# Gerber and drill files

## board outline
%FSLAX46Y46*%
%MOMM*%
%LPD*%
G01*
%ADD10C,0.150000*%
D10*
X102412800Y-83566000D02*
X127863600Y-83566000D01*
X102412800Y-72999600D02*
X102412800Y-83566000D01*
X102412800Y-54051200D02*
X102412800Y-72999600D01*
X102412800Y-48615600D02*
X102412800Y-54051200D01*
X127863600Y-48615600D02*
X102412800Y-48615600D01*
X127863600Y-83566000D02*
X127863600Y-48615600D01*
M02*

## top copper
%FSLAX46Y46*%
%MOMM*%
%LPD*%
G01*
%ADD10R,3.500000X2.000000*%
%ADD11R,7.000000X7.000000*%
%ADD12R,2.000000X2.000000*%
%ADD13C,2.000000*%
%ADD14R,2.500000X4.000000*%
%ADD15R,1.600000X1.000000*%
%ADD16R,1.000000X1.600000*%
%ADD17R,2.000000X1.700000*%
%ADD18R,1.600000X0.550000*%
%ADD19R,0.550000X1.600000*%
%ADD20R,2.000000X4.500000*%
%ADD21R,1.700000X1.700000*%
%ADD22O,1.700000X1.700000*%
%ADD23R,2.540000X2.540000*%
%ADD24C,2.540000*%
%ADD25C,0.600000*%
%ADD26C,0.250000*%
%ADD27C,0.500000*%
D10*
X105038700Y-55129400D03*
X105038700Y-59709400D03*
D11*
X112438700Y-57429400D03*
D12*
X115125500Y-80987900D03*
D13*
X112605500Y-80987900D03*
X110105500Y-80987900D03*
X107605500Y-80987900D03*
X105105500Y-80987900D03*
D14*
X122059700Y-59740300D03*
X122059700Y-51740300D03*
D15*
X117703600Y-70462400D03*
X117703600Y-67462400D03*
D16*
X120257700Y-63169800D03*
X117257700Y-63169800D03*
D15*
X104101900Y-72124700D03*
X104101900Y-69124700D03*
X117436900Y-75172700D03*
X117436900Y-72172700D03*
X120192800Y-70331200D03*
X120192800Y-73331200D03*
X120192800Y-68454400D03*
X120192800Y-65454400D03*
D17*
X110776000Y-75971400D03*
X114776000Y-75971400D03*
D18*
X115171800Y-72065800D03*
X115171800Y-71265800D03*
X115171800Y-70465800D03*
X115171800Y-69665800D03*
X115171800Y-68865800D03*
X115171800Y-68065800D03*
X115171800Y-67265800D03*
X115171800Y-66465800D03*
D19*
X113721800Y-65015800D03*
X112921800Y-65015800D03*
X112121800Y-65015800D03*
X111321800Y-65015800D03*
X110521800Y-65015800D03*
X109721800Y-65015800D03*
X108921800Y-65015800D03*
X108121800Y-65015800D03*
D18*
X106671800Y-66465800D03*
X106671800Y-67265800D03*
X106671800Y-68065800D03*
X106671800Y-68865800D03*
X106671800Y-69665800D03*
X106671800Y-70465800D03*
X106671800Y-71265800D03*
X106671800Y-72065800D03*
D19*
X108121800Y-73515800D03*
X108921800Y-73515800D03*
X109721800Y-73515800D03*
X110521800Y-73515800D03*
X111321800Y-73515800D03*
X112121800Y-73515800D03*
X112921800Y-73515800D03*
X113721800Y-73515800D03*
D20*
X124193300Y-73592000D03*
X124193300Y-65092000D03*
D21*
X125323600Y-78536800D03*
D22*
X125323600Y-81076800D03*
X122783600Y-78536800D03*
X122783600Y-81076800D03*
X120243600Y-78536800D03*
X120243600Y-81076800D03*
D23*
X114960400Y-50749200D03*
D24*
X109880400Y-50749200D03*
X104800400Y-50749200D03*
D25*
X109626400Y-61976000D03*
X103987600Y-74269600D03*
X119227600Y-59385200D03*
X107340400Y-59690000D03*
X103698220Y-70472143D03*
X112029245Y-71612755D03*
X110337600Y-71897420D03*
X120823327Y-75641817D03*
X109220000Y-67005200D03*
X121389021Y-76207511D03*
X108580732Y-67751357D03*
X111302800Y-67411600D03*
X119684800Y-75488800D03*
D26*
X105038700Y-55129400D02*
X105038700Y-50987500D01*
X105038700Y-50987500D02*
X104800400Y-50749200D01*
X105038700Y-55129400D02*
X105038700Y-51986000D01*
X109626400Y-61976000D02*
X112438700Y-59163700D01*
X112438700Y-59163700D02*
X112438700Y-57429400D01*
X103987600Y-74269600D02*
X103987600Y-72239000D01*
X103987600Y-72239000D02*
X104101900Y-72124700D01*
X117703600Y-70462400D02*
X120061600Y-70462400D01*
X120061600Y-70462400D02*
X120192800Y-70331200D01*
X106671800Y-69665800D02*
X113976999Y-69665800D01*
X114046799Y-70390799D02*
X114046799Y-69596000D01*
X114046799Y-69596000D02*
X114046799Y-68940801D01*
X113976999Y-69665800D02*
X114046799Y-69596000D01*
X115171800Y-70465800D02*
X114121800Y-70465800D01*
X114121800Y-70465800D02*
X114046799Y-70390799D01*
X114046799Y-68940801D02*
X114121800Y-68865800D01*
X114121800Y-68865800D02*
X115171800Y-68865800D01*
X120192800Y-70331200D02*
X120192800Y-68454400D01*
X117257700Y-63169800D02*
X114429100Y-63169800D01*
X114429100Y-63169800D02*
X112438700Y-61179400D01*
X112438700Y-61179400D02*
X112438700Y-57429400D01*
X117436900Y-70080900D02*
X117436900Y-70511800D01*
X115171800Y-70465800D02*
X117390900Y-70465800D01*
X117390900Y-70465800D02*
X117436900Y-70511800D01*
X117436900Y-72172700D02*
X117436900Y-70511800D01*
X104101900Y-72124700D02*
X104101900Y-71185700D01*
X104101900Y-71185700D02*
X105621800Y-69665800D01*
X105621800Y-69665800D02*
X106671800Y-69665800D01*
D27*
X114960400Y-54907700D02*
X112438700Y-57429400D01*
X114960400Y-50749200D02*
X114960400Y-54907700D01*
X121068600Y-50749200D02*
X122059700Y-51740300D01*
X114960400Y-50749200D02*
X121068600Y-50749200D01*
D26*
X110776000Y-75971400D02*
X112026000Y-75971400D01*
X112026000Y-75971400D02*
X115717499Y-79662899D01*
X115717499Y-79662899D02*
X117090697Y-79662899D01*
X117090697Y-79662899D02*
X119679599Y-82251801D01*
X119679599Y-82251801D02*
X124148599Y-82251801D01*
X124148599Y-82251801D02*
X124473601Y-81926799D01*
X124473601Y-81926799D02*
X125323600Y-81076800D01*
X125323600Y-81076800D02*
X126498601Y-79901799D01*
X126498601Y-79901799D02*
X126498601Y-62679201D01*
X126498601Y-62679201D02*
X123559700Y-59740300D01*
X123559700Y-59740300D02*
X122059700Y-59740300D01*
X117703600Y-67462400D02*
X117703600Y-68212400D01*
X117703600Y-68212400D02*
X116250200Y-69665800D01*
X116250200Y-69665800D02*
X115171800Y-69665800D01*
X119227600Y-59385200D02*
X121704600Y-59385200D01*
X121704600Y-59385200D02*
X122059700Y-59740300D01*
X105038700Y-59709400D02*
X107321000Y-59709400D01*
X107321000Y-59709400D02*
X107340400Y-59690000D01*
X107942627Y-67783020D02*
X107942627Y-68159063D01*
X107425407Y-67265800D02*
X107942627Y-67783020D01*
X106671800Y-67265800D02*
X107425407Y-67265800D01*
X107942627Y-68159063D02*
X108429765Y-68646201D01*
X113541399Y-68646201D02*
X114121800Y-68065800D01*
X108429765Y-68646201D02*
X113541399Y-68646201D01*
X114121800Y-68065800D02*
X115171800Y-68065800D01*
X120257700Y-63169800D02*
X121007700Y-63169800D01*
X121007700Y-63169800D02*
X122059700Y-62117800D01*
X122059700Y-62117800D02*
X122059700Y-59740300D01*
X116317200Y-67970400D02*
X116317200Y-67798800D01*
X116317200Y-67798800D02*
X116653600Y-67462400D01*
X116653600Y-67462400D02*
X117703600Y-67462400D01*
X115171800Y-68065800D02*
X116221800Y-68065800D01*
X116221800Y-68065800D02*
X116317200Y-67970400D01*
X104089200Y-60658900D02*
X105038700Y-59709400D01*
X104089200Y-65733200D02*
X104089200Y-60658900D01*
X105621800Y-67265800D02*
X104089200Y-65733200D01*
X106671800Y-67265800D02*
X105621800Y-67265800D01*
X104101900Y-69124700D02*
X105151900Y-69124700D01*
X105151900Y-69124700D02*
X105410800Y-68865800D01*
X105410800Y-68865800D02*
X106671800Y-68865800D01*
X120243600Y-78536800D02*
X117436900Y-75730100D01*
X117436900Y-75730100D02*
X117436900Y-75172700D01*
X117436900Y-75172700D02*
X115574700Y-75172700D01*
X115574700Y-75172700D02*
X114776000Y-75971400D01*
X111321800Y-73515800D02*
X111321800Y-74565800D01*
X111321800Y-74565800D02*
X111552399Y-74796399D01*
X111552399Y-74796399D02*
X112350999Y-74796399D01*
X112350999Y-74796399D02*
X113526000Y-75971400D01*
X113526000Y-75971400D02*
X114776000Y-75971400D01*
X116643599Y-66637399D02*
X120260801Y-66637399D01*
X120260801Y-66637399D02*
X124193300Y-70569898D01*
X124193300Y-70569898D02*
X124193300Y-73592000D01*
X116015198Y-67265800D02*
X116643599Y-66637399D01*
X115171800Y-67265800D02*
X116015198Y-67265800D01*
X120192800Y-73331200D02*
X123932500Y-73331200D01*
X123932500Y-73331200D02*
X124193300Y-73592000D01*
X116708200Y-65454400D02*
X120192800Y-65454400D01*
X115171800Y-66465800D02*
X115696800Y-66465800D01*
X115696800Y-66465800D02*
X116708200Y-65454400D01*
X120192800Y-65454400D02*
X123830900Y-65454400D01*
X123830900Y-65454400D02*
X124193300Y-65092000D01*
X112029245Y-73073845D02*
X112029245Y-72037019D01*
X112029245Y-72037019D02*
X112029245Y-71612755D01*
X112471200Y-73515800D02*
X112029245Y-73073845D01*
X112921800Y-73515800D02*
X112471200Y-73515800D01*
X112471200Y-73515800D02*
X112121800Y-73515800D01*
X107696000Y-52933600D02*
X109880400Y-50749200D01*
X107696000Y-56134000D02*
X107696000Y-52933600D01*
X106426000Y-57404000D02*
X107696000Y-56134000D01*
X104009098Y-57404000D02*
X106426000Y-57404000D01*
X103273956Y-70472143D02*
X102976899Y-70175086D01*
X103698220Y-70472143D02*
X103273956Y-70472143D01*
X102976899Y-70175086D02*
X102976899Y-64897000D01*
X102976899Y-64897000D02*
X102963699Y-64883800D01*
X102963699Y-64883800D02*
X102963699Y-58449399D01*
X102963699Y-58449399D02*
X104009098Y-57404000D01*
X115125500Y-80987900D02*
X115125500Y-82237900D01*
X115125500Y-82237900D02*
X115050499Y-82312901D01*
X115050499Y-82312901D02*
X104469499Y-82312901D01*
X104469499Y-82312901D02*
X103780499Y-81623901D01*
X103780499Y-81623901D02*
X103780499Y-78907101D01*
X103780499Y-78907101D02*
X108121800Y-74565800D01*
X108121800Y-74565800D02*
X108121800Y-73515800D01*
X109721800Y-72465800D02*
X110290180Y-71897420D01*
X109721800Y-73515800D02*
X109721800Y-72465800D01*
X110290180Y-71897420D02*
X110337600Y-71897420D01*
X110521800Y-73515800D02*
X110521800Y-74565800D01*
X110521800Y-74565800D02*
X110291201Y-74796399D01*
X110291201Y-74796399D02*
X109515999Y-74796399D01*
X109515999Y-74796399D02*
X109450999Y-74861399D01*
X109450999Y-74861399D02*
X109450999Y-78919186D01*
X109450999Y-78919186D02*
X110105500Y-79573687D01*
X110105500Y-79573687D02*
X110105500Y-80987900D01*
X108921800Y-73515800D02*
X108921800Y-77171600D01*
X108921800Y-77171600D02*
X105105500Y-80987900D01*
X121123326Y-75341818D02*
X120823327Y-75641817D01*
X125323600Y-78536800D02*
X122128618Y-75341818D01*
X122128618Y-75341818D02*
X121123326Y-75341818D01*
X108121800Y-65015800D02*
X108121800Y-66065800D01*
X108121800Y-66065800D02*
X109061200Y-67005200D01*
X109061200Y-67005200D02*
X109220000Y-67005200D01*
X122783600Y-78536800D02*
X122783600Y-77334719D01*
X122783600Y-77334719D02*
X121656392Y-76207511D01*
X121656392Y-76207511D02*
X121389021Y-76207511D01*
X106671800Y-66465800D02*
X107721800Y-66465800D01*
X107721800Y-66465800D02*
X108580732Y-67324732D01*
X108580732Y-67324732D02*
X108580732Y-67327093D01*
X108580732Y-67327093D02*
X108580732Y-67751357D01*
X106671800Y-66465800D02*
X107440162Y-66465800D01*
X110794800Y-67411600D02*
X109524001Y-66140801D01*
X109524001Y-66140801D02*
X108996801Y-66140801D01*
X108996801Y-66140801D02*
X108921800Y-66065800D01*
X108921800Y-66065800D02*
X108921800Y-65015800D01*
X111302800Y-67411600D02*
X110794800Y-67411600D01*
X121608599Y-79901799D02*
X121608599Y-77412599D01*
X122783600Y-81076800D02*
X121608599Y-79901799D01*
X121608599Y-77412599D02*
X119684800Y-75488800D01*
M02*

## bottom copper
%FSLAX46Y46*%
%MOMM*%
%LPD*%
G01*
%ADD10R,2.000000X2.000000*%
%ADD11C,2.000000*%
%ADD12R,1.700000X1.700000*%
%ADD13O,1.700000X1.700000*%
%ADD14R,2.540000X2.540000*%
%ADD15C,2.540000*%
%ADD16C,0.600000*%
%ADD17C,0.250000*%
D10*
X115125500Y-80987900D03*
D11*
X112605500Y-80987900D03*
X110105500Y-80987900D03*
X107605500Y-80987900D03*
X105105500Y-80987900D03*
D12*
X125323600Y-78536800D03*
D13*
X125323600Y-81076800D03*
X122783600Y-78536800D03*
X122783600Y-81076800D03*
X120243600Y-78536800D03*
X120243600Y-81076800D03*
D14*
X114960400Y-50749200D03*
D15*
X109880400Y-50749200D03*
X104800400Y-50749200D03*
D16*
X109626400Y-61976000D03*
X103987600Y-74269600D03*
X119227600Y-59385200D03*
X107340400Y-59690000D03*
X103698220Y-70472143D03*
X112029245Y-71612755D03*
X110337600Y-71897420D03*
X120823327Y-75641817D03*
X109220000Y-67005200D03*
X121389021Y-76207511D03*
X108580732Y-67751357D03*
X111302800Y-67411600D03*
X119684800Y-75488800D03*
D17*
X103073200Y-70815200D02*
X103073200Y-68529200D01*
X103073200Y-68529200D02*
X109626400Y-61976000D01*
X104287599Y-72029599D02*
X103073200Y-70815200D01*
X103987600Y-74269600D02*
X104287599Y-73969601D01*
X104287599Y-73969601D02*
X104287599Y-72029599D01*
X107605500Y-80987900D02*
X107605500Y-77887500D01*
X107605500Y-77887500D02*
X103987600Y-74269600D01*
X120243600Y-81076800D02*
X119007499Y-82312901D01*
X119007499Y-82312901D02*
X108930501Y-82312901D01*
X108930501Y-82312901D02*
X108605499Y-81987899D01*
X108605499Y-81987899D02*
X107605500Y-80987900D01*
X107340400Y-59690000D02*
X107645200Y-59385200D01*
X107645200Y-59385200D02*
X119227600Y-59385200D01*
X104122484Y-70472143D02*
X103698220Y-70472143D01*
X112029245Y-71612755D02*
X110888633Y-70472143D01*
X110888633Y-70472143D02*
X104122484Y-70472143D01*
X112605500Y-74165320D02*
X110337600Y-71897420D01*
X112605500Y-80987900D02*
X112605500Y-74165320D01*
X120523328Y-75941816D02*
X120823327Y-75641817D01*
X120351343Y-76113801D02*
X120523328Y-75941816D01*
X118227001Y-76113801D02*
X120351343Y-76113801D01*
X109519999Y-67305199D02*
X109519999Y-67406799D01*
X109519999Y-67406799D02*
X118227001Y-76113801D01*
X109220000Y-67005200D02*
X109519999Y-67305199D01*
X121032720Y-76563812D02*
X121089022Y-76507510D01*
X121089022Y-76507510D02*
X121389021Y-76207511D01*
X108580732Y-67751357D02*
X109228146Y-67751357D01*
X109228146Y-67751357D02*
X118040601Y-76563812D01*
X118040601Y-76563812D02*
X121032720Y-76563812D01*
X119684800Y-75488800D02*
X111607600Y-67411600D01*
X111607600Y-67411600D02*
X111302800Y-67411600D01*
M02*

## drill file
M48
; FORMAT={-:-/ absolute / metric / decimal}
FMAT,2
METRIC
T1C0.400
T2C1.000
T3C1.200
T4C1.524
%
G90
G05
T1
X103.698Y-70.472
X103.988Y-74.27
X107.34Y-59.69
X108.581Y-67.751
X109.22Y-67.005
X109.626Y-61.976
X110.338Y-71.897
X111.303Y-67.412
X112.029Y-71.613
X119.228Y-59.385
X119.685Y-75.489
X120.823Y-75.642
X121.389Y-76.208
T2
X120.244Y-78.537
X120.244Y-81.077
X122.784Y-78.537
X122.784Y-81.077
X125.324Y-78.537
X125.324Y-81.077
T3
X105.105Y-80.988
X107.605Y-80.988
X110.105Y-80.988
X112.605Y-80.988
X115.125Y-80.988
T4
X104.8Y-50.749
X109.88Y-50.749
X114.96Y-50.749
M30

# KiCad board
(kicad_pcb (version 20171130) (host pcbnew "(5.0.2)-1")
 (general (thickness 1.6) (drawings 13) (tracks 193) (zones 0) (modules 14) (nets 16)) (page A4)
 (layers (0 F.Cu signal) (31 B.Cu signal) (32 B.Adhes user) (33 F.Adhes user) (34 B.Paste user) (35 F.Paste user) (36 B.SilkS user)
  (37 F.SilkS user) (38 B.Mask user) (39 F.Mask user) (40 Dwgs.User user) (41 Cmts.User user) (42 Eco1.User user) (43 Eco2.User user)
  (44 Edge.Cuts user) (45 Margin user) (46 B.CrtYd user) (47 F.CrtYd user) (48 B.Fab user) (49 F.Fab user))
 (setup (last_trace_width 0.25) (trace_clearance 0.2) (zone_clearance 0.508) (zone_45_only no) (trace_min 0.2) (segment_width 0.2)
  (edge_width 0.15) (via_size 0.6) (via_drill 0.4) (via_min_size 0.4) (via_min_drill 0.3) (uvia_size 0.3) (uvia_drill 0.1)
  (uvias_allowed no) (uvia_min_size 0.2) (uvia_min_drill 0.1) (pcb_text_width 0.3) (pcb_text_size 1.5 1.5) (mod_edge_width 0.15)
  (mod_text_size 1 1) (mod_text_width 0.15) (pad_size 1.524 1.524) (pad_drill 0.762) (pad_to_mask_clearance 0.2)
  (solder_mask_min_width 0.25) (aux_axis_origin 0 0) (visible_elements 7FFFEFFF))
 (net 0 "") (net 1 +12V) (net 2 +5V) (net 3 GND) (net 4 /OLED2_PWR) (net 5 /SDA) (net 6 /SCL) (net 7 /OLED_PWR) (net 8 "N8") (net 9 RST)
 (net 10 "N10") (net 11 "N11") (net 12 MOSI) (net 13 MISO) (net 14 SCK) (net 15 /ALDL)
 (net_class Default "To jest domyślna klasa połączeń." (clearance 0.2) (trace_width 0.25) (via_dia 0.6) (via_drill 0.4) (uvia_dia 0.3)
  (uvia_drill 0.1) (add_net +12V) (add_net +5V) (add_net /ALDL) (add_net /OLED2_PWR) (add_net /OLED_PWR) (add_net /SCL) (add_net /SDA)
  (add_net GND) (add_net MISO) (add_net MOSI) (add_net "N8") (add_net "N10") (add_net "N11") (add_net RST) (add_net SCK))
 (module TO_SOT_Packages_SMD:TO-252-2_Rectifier (layer F.Cu) (at 109.6137 57.4294)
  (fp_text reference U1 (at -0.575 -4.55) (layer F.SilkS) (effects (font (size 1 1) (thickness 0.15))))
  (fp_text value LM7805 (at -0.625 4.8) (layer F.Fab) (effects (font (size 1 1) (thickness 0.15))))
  (pad 1 smd rect (at -4.575 -2.3 270) (size 2 3.5) (layers F.Cu F.Paste F.Mask) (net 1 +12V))
  (pad 3 smd rect (at -4.575 2.28 270) (size 2 3.5) (layers F.Cu F.Paste F.Mask) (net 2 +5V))
  (pad 2 smd rect (at 2.825 0 270) (size 7 7) (layers F.Cu F.Paste F.Mask) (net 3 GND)))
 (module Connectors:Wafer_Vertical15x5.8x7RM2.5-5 (layer F.Cu) (at 115.1255 80.9879 180)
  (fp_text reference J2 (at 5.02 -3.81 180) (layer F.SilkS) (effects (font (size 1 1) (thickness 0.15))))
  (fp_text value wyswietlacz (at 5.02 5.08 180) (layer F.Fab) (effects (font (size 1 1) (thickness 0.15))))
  (pad 1 thru_hole rect (at 0 0 180) (size 2 2) (drill 1.2) (layers *.Cu *.Mask) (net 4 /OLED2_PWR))
  (pad 2 thru_hole circle (at 2.52 0 180) (size 2 2) (drill 1.2) (layers *.Cu *.Mask) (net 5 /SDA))
  (pad 3 thru_hole circle (at 5.02 0 180) (size 2 2) (drill 1.2) (layers *.Cu *.Mask) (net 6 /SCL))
  (pad 4 thru_hole circle (at 7.52 0 180) (size 2 2) (drill 1.2) (layers *.Cu *.Mask) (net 3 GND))
  (pad 5 thru_hole circle (at 10.02 0 180) (size 2 2) (drill 1.2) (layers *.Cu *.Mask) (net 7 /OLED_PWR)))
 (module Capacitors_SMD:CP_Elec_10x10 (layer F.Cu) (at 122.0597 55.7403 90)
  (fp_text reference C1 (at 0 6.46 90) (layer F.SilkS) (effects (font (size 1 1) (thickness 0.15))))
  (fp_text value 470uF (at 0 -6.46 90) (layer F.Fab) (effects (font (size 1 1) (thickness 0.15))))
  (pad 1 smd rect (at -4 0 270) (size 4 2.5) (layers F.Cu F.Paste F.Mask) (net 2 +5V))
  (pad 2 smd rect (at 4 0 270) (size 4 2.5) (layers F.Cu F.Paste F.Mask) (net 3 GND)))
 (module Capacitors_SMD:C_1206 (layer F.Cu) (at 117.7036 68.9624 90)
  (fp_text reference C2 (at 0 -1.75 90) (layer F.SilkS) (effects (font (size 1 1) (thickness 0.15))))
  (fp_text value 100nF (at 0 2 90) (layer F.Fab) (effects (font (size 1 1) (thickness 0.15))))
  (pad 1 smd rect (at -1.5 0 90) (size 1 1.6) (layers F.Cu F.Paste F.Mask) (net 3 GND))
  (pad 2 smd rect (at 1.5 0 90) (size 1 1.6) (layers F.Cu F.Paste F.Mask) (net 2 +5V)))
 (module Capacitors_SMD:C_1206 (layer F.Cu) (at 118.7577 63.1698 180)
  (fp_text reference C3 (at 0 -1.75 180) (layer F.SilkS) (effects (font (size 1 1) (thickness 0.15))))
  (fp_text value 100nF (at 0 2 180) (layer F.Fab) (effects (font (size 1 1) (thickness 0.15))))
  (pad 1 smd rect (at -1.5 0 180) (size 1 1.6) (layers F.Cu F.Paste F.Mask) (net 2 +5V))
  (pad 2 smd rect (at 1.5 0 180) (size 1 1.6) (layers F.Cu F.Paste F.Mask) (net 3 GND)))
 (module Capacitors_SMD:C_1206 (layer F.Cu) (at 104.1019 70.6247 90)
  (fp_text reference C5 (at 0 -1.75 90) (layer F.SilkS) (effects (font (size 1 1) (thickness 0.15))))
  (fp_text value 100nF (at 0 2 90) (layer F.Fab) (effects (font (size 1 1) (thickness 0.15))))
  (pad 1 smd rect (at -1.5 0 90) (size 1 1.6) (layers F.Cu F.Paste F.Mask) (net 3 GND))
  (pad 2 smd rect (at 1.5 0 90) (size 1 1.6) (layers F.Cu F.Paste F.Mask) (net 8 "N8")))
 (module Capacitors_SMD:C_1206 (layer F.Cu) (at 117.4369 73.6727 90)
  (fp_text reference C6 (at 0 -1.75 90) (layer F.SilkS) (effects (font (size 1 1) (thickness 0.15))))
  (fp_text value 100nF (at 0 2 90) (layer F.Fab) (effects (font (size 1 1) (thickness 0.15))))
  (pad 1 smd rect (at -1.5 0 90) (size 1 1.6) (layers F.Cu F.Paste F.Mask) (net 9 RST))
  (pad 2 smd rect (at 1.5 0 90) (size 1 1.6) (layers F.Cu F.Paste F.Mask) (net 3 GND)))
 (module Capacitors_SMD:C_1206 (layer F.Cu) (at 120.1928 71.8312 270)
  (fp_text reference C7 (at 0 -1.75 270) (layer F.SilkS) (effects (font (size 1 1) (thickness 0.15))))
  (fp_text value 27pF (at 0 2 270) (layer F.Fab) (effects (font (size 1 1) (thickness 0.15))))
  (pad 1 smd rect (at -1.5 0 270) (size 1 1.6) (layers F.Cu F.Paste F.Mask) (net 3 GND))
  (pad 2 smd rect (at 1.5 0 270) (size 1 1.6) (layers F.Cu F.Paste F.Mask) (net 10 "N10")))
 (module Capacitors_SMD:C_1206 (layer F.Cu) (at 120.1928 66.9544 90)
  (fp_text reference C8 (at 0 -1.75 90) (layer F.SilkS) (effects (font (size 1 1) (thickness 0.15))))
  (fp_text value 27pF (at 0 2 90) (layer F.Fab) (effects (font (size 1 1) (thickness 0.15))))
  (pad 1 smd rect (at -1.5 0 90) (size 1 1.6) (layers F.Cu F.Paste F.Mask) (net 3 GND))
  (pad 2 smd rect (at 1.5 0 90) (size 1 1.6) (layers F.Cu F.Paste F.Mask) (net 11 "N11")))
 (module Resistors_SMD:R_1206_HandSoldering (layer F.Cu) (at 112.776 75.9714)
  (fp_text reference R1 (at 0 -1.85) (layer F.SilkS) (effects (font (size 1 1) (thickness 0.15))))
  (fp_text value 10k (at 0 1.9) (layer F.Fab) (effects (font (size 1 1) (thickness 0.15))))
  (pad 1 smd rect (at -2 0) (size 2 1.7) (layers F.Cu F.Paste F.Mask) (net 2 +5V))
  (pad 2 smd rect (at 2 0) (size 2 1.7) (layers F.Cu F.Paste F.Mask) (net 9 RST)))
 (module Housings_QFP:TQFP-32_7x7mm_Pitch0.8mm (layer F.Cu) (at 110.9218 69.2658 180)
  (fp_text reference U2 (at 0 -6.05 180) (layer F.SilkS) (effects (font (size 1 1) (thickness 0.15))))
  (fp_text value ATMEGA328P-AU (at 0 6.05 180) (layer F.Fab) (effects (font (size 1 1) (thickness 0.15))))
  (pad 1 smd rect (at -4.25 -2.8 180) (size 1.6 0.55) (layers F.Cu F.Paste F.Mask))
  (pad 2 smd rect (at -4.25 -2 180) (size 1.6 0.55) (layers F.Cu F.Paste F.Mask))
  (pad 3 smd rect (at -4.25 -1.2 180) (size 1.6 0.55) (layers F.Cu F.Paste F.Mask) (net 3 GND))
  (pad 4 smd rect (at -4.25 -0.4 180) (size 1.6 0.55) (layers F.Cu F.Paste F.Mask) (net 2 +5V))
  (pad 5 smd rect (at -4.25 0.4 180) (size 1.6 0.55) (layers F.Cu F.Paste F.Mask) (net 3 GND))
  (pad 6 smd rect (at -4.25 1.2 180) (size 1.6 0.55) (layers F.Cu F.Paste F.Mask) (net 2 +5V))
  (pad 7 smd rect (at -4.25 2 180) (size 1.6 0.55) (layers F.Cu F.Paste F.Mask) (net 10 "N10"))
  (pad 8 smd rect (at -4.25 2.8 180) (size 1.6 0.55) (layers F.Cu F.Paste F.Mask) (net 11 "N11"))
  (pad 9 smd rect (at -2.8 4.25 270) (size 1.6 0.55) (layers F.Cu F.Paste F.Mask))
  (pad 10 smd rect (at -2 4.25 270) (size 1.6 0.55) (layers F.Cu F.Paste F.Mask))
  (pad 11 smd rect (at -1.2 4.25 270) (size 1.6 0.55) (layers F.Cu F.Paste F.Mask))
  (pad 12 smd rect (at -0.4 4.25 270) (size 1.6 0.55) (layers F.Cu F.Paste F.Mask))
  (pad 13 smd rect (at 0.4 4.25 270) (size 1.6 0.55) (layers F.Cu F.Paste F.Mask))
  (pad 14 smd rect (at 1.2 4.25 270) (size 1.6 0.55) (layers F.Cu F.Paste F.Mask))
  (pad 15 smd rect (at 2 4.25 270) (size 1.6 0.55) (layers F.Cu F.Paste F.Mask) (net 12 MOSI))
  (pad 16 smd rect (at 2.8 4.25 270) (size 1.6 0.55) (layers F.Cu F.Paste F.Mask) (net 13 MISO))
  (pad 17 smd rect (at 4.25 2.8 180) (size 1.6 0.55) (layers F.Cu F.Paste F.Mask) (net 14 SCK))
  (pad 18 smd rect (at 4.25 2 180) (size 1.6 0.55) (layers F.Cu F.Paste F.Mask) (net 2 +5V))
  (pad 19 smd rect (at 4.25 1.2 180) (size 1.6 0.55) (layers F.Cu F.Paste F.Mask))
  (pad 20 smd rect (at 4.25 0.4 180) (size 1.6 0.55) (layers F.Cu F.Paste F.Mask) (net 8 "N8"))
  (pad 21 smd rect (at 4.25 -0.4 180) (size 1.6 0.55) (layers F.Cu F.Paste F.Mask) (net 3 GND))
  (pad 22 smd rect (at 4.25 -1.2 180) (size 1.6 0.55) (layers F.Cu F.Paste F.Mask))
  (pad 23 smd rect (at 4.25 -2 180) (size 1.6 0.55) (layers F.Cu F.Paste F.Mask))
  (pad 24 smd rect (at 4.25 -2.8 180) (size 1.6 0.55) (layers F.Cu F.Paste F.Mask))
  (pad 25 smd rect (at 2.8 -4.25 270) (size 1.6 0.55) (layers F.Cu F.Paste F.Mask) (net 4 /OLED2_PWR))
  (pad 26 smd rect (at 2 -4.25 270) (size 1.6 0.55) (layers F.Cu F.Paste F.Mask) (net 7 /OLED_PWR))
  (pad 27 smd rect (at 1.2 -4.25 270) (size 1.6 0.55) (layers F.Cu F.Paste F.Mask) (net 5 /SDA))
  (pad 28 smd rect (at 0.4 -4.25 270) (size 1.6 0.55) (layers F.Cu F.Paste F.Mask) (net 6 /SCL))
  (pad 29 smd rect (at -0.4 -4.25 270) (size 1.6 0.55) (layers F.Cu F.Paste F.Mask) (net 9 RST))
  (pad 30 smd rect (at -1.2 -4.25 270) (size 1.6 0.55) (layers F.Cu F.Paste F.Mask) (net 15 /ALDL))
  (pad 31 smd rect (at -2 -4.25 270) (size 1.6 0.55) (layers F.Cu F.Paste F.Mask) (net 15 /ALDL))
  (pad 32 smd rect (at -2.8 -4.25 270) (size 1.6 0.55) (layers F.Cu F.Paste F.Mask)))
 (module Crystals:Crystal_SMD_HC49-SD (layer F.Cu) (at 124.1933 69.342 90)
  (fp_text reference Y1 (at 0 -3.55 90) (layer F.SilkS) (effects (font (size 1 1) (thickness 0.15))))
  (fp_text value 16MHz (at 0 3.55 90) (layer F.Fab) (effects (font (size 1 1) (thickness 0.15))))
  (pad 1 smd rect (at -4.25 0 90) (size 4.5 2) (layers F.Cu F.Paste F.Mask) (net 10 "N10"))
  (pad 2 smd rect (at 4.25 0 90) (size 4.5 2) (layers F.Cu F.Paste F.Mask) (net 11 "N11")))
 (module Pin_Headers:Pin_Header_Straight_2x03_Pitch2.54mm (layer F.Cu) (at 125.3236 78.5368 270)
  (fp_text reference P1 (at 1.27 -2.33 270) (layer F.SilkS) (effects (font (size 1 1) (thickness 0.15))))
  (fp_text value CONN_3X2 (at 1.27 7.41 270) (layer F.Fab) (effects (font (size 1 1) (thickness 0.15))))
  (pad 1 thru_hole rect (at 0 0 270) (size 1.7 1.7) (drill 1) (layers *.Cu *.Mask) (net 13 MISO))
  (pad 2 thru_hole oval (at 2.54 0 270) (size 1.7 1.7) (drill 1) (layers *.Cu *.Mask) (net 2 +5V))
  (pad 3 thru_hole oval (at 0 2.54 270) (size 1.7 1.7) (drill 1) (layers *.Cu *.Mask) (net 14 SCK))
  (pad 4 thru_hole oval (at 2.54 2.54 270) (size 1.7 1.7) (drill 1) (layers *.Cu *.Mask) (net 12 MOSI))
  (pad 5 thru_hole oval (at 0 5.08 270) (size 1.7 1.7) (drill 1) (layers *.Cu *.Mask) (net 9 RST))
  (pad 6 thru_hole oval (at 2.54 5.08 270) (size 1.7 1.7) (drill 1) (layers *.Cu *.Mask) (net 3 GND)))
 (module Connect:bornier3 (layer F.Cu) (at 109.8804 50.7492 180)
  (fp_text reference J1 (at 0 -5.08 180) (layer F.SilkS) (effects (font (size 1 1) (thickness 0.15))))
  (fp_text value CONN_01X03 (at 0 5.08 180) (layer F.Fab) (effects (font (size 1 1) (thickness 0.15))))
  (pad 1 thru_hole rect (at -5.08 0 180) (size 2.54 2.54) (drill 1.524) (layers *.Cu *.Mask F.SilkS) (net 3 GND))
  (pad 2 thru_hole circle (at 0 0 180) (size 2.54 2.54) (drill 1.524) (layers *.Cu *.Mask F.SilkS) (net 15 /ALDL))
  (pad 3 thru_hole circle (at 5.08 0 180) (size 2.54 2.54) (drill 1.524) (layers *.Cu *.Mask F.SilkS) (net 1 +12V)))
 (gr_line (start 102.4128 83.566) (end 127.8636 83.566) (angle 90) (layer Edge.Cuts) (width 0.15))
 (gr_line (start 102.4128 72.9996) (end 102.4128 83.566) (angle 90) (layer Edge.Cuts) (width 0.15))
 (gr_line (start 102.4128 54.0512) (end 102.4128 72.9996) (angle 90) (layer Edge.Cuts) (width 0.15))
 (gr_line (start 102.4128 48.6156) (end 102.4128 54.0512) (angle 90) (layer Edge.Cuts) (width 0.15))
 (gr_line (start 127.8636 48.6156) (end 102.4128 48.6156) (angle 90) (layer Edge.Cuts) (width 0.15))
 (gr_line (start 127.8636 83.566) (end 127.8636 48.6156) (angle 90) (layer Edge.Cuts) (width 0.15))
 (segment (start 105.0387 55.1294) (end 105.0387 50.9875) (width 0.25) (layer F.Cu) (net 1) (status 30))
 (segment (start 105.0387 50.9875) (end 104.8004 50.7492) (width 0.25) (layer F.Cu) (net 1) (status 30))
 (segment (start 105.0387 55.1294) (end 105.0387 51.986) (width 0.25) (layer F.Cu) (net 1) (status 30))
 (segment (start 109.6264 61.976) (end 112.4387 59.1637) (width 0.25) (layer F.Cu) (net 3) (status 20))
 (segment (start 112.4387 59.1637) (end 112.4387 57.4294) (width 0.25) (layer F.Cu) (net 3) (status 30))
 (segment (start 103.0732 70.8152) (end 103.0732 68.5292) (width 0.25) (layer B.Cu) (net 3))
 (segment (start 103.0732 68.5292) (end 109.6264 61.976) (width 0.25) (layer B.Cu) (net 3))
 (via (at 109.6264 61.976) (size 0.6) (drill 0.4) (layers F.Cu B.Cu) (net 3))
 (segment (start 104.287599 72.029599) (end 103.0732 70.8152) (width 0.25) (layer B.Cu) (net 3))
 (segment (start 103.9876 74.2696) (end 104.287599 73.969601) (width 0.25) (layer B.Cu) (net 3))
 (segment (start 104.287599 73.969601) (end 104.287599 72.029599) (width 0.25) (layer B.Cu) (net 3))
 (segment (start 103.9876 74.2696) (end 103.9876 72.239) (width 0.25) (layer F.Cu) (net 3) (status 20))
 (segment (start 103.9876 72.239) (end 104.1019 72.1247) (width 0.25) (layer F.Cu) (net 3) (status 30))
 (segment (start 107.6055 80.9879) (end 107.6055 77.8875) (width 0.25) (layer B.Cu) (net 3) (status 10))
 (segment (start 107.6055 77.8875) (end 103.9876 74.2696) (width 0.25) (layer B.Cu) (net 3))
 (via (at 103.9876 74.2696) (size 0.6) (drill 0.4) (layers F.Cu B.Cu) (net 3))
 (segment (start 120.2436 81.0768) (end 119.007499 82.312901) (width 0.25) (layer B.Cu) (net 3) (status 10))
 (segment (start 119.007499 82.312901) (end 108.930501 82.312901) (width 0.25) (layer B.Cu) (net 3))
 (segment (start 108.930501 82.312901) (end 108.605499 81.987899) (width 0.25) (layer B.Cu) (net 3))
 (segment (start 108.605499 81.987899) (end 107.6055 80.9879) (width 0.25) (layer B.Cu) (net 3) (status 20))
 (segment (start 117.7036 70.4624) (end 120.0616 70.4624) (width 0.25) (layer F.Cu) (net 3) (status 30))
 (segment (start 120.0616 70.4624) (end 120.1928 70.3312) (width 0.25) (layer F.Cu) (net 3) (status 30))
 (segment (start 106.6718 69.6658) (end 113.976999 69.6658) (width 0.25) (layer F.Cu) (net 3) (status 10))
 (segment (start 114.046799 70.390799) (end 114.046799 69.596) (width 0.25) (layer F.Cu) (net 3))
 (segment (start 114.046799 69.596) (end 114.046799 68.940801) (width 0.25) (layer F.Cu) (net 3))
 (segment (start 113.976999 69.6658) (end 114.046799 69.596) (width 0.25) (layer F.Cu) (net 3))
 (segment (start 115.1718 70.4658) (end 114.1218 70.4658) (width 0.25) (layer F.Cu) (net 3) (status 10))
 (segment (start 114.1218 70.4658) (end 114.046799 70.390799) (width 0.25) (layer F.Cu) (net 3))
 (segment (start 114.046799 68.940801) (end 114.1218 68.8658) (width 0.25) (layer F.Cu) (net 3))
 (segment (start 114.1218 68.8658) (end 115.1718 68.8658) (width 0.25) (layer F.Cu) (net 3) (status 20))
 (segment (start 120.1928 70.3312) (end 120.1928 68.4544) (width 0.25) (layer F.Cu) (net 3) (status 30))
 (segment (start 117.2577 63.1698) (end 114.4291 63.1698) (width 0.25) (layer F.Cu) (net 3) (status 10))
 (segment (start 114.4291 63.1698) (end 112.4387 61.1794) (width 0.25) (layer F.Cu) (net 3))
 (segment (start 112.4387 61.1794) (end 112.4387 57.4294) (width 0.25) (layer F.Cu) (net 3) (status 20))
 (segment (start 117.4369 70.0809) (end 117.4369 70.5118) (width 0.25) (layer F.Cu) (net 3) (status 30))
 (segment (start 115.1718 70.4658) (end 117.3909 70.4658) (width 0.25) (layer F.Cu) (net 3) (status 30))
 (segment (start 117.3909 70.4658) (end 117.4369 70.5118) (width 0.25) (layer F.Cu) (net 3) (status 30))
 (segment (start 117.4369 72.1727) (end 117.4369 70.5118) (width 0.25) (layer F.Cu) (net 3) (status 30))
 (segment (start 104.1019 72.1247) (end 104.1019 71.1857) (width 0.25) (layer F.Cu) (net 3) (status 10))
 (segment (start 104.1019 71.1857) (end 105.6218 69.6658) (width 0.25) (layer F.Cu) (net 3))
 (segment (start 105.6218 69.6658) (end 106.6718 69.6658) (width 0.25) (layer F.Cu) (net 3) (status 20))
 (segment (start 114.9604 54.9077) (end 112.4387 57.4294) (width 0.5) (layer F.Cu) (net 3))
 (segment (start 114.9604 50.7492) (end 114.9604 54.9077) (width 0.5) (layer F.Cu) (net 3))
 (segment (start 121.0686 50.7492) (end 122.0597 51.7403) (width 0.5) (layer F.Cu) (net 3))
 (segment (start 114.9604 50.7492) (end 121.0686 50.7492) (width 0.5) (layer F.Cu) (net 3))
 (segment (start 110.776 75.9714) (end 112.026 75.9714) (width 0.25) (layer F.Cu) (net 2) (status 10))
 (segment (start 112.026 75.9714) (end 115.717499 79.662899) (width 0.25) (layer F.Cu) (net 2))
 (segment (start 115.717499 79.662899) (end 117.090697 79.662899) (width 0.25) (layer F.Cu) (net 2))
 (segment (start 117.090697 79.662899) (end 119.679599 82.251801) (width 0.25) (layer F.Cu) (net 2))
 (segment (start 119.679599 82.251801) (end 124.148599 82.251801) (width 0.25) (layer F.Cu) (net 2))
 (segment (start 124.148599 82.251801) (end 124.473601 81.926799) (width 0.25) (layer F.Cu) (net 2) (status 20))
 (segment (start 124.473601 81.926799) (end 125.3236 81.0768) (width 0.25) (layer F.Cu) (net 2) (status 30))
 (segment (start 125.3236 81.0768) (end 126.498601 79.901799) (width 0.25) (layer F.Cu) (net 2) (status 10))
 (segment (start 126.498601 79.901799) (end 126.498601 62.679201) (width 0.25) (layer F.Cu) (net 2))
 (segment (start 126.498601 62.679201) (end 123.5597 59.7403) (width 0.25) (layer F.Cu) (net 2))
 (segment (start 123.5597 59.7403) (end 122.0597 59.7403) (width 0.25) (layer F.Cu) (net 2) (status 20))
 (segment (start 117.7036 67.4624) (end 117.7036 68.2124) (width 0.25) (layer F.Cu) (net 2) (status 10))
 (segment (start 117.7036 68.2124) (end 116.2502 69.6658) (width 0.25) (layer F.Cu) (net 2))
 (segment (start 116.2502 69.6658) (end 115.1718 69.6658) (width 0.25) (layer F.Cu) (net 2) (status 20))
 (segment (start 119.2276 59.3852) (end 121.7046 59.3852) (width 0.25) (layer F.Cu) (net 2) (status 20))
 (segment (start 121.7046 59.3852) (end 122.0597 59.7403) (width 0.25) (layer F.Cu) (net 2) (status 30))
 (segment (start 107.3404 59.69) (end 107.6452 59.3852) (width 0.25) (layer B.Cu) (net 2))
 (via (at 119.2276 59.3852) (size 0.6) (drill 0.4) (layers F.Cu B.Cu) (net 2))
 (segment (start 107.6452 59.3852) (end 119.2276 59.3852) (width 0.25) (layer B.Cu) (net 2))
 (segment (start 105.0387 59.7094) (end 107.321 59.7094) (width 0.25) (layer F.Cu) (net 2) (status 10))
 (segment (start 107.321 59.7094) (end 107.3404 59.69) (width 0.25) (layer F.Cu) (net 2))
 (via (at 107.3404 59.69) (size 0.6) (drill 0.4) (layers F.Cu B.Cu) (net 2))
 (segment (start 107.942627 67.78302) (end 107.942627 68.159063) (width 0.25) (layer F.Cu) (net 2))
 (segment (start 107.425407 67.2658) (end 107.942627 67.78302) (width 0.25) (layer F.Cu) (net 2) (status 10))
 (segment (start 106.6718 67.2658) (end 107.425407 67.2658) (width 0.25) (layer F.Cu) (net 2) (status 30))
 (segment (start 107.942627 68.159063) (end 108.429765 68.646201) (width 0.25) (layer F.Cu) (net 2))
 (segment (start 113.541399 68.646201) (end 114.1218 68.0658) (width 0.25) (layer F.Cu) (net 2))
 (segment (start 108.429765 68.646201) (end 113.541399 68.646201) (width 0.25) (layer F.Cu) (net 2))
 (segment (start 114.1218 68.0658) (end 115.1718 68.0658) (width 0.25) (layer F.Cu) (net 2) (status 20))
 (segment (start 120.2577 63.1698) (end 121.0077 63.1698) (width 0.25) (layer F.Cu) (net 2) (status 10))
 (segment (start 121.0077 63.1698) (end 122.0597 62.1178) (width 0.25) (layer F.Cu) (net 2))
 (segment (start 122.0597 62.1178) (end 122.0597 59.7403) (width 0.25) (layer F.Cu) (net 2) (status 20))
 (segment (start 116.3172 67.9704) (end 116.3172 67.7988) (width 0.25) (layer F.Cu) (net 2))
 (segment (start 116.3172 67.7988) (end 116.6536 67.4624) (width 0.25) (layer F.Cu) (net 2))
 (segment (start 116.6536 67.4624) (end 117.7036 67.4624) (width 0.25) (layer F.Cu) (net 2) (status 20))
 (segment (start 115.1718 68.0658) (end 116.2218 68.0658) (width 0.25) (layer F.Cu) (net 2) (status 10))
 (segment (start 116.2218 68.0658) (end 116.3172 67.9704) (width 0.25) (layer F.Cu) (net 2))
 (segment (start 104.0892 60.6589) (end 105.0387 59.7094) (width 0.25) (layer F.Cu) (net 2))
 (segment (start 104.0892 65.7332) (end 104.0892 60.6589) (width 0.25) (layer F.Cu) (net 2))
 (segment (start 105.6218 67.2658) (end 104.0892 65.7332) (width 0.25) (layer F.Cu) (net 2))
 (segment (start 106.6718 67.2658) (end 105.6218 67.2658) (width 0.25) (layer F.Cu) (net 2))
 (segment (start 104.1019 69.1247) (end 105.1519 69.1247) (width 0.25) (layer F.Cu) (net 8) (status 10))
 (segment (start 105.1519 69.1247) (end 105.4108 68.8658) (width 0.25) (layer F.Cu) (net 8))
 (segment (start 105.4108 68.8658) (end 106.6718 68.8658) (width 0.25) (layer F.Cu) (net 8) (status 20))
 (segment (start 120.2436 78.5368) (end 117.4369 75.7301) (width 0.25) (layer F.Cu) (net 9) (status 10))
 (segment (start 117.4369 75.7301) (end 117.4369 75.1727) (width 0.25) (layer F.Cu) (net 9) (status 20))
 (segment (start 117.4369 75.1727) (end 115.5747 75.1727) (width 0.25) (layer F.Cu) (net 9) (status 30))
 (segment (start 115.5747 75.1727) (end 114.776 75.9714) (width 0.25) (layer F.Cu) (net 9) (status 30))
 (segment (start 111.3218 73.5158) (end 111.3218 74.5658) (width 0.25) (layer F.Cu) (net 9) (status 10))
 (segment (start 111.3218 74.5658) (end 111.552399 74.796399) (width 0.25) (layer F.Cu) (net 9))
 (segment (start 111.552399 74.796399) (end 112.350999 74.796399) (width 0.25) (layer F.Cu) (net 9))
 (segment (start 112.350999 74.796399) (end 113.526 75.9714) (width 0.25) (layer F.Cu) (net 9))
 (segment (start 113.526 75.9714) (end 114.776 75.9714) (width 0.25) (layer F.Cu) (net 9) (status 20))
 (segment (start 116.643599 66.637399) (end 120.260801 66.637399) (width 0.25) (layer F.Cu) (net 10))
 (segment (start 120.260801 66.637399) (end 124.1933 70.569898) (width 0.25) (layer F.Cu) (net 10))
 (segment (start 124.1933 70.569898) (end 124.1933 73.592) (width 0.25) (layer F.Cu) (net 10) (status 20))
 (segment (start 116.015198 67.2658) (end 116.643599 66.637399) (width 0.25) (layer F.Cu) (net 10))
 (segment (start 115.1718 67.2658) (end 116.015198 67.2658) (width 0.25) (layer F.Cu) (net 10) (status 10))
 (segment (start 120.1928 73.3312) (end 123.9325 73.3312) (width 0.25) (layer F.Cu) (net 10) (status 30))
 (segment (start 123.9325 73.3312) (end 124.1933 73.592) (width 0.25) (layer F.Cu) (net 10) (status 30))
 (segment (start 116.7082 65.4544) (end 120.1928 65.4544) (width 0.25) (layer F.Cu) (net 11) (status 20))
 (segment (start 115.1718 66.4658) (end 115.6968 66.4658) (width 0.25) (layer F.Cu) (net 11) (status 30))
 (segment (start 115.6968 66.4658) (end 116.7082 65.4544) (width 0.25) (layer F.Cu) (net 11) (status 10))
 (segment (start 120.1928 65.4544) (end 123.8309 65.4544) (width 0.25) (layer F.Cu) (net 11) (status 30))
 (segment (start 123.8309 65.4544) (end 124.1933 65.092) (width 0.25) (layer F.Cu) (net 11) (status 30))
 (segment (start 104.122484 70.472143) (end 103.69822 70.472143) (width 0.25) (layer B.Cu) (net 15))
 (segment (start 112.029245 71.612755) (end 110.888633 70.472143) (width 0.25) (layer B.Cu) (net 15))
 (segment (start 110.888633 70.472143) (end 104.122484 70.472143) (width 0.25) (layer B.Cu) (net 15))
 (via (at 103.69822 70.472143) (size 0.6) (drill 0.4) (layers F.Cu B.Cu) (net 15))
 (segment (start 112.029245 73.073845) (end 112.029245 72.037019) (width 0.25) (layer F.Cu) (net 15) (status 10))
 (segment (start 112.029245 72.037019) (end 112.029245 71.612755) (width 0.25) (layer F.Cu) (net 15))
 (via (at 112.029245 71.612755) (size 0.6) (drill 0.4) (layers F.Cu B.Cu) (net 15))
 (segment (start 112.4712 73.5158) (end 112.029245 73.073845) (width 0.25) (layer F.Cu) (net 15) (status 20))
 (segment (start 112.9218 73.5158) (end 112.4712 73.5158) (width 0.25) (layer F.Cu) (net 15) (status 10))
 (segment (start 112.4712 73.5158) (end 112.1218 73.5158) (width 0.25) (layer F.Cu) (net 15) (status 20))
 (segment (start 107.696 52.9336) (end 109.8804 50.7492) (width 0.25) (layer F.Cu) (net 15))
 (segment (start 107.696 56.134) (end 107.696 52.9336) (width 0.25) (layer F.Cu) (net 15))
 (segment (start 106.426 57.404) (end 107.696 56.134) (width 0.25) (layer F.Cu) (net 15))
 (segment (start 104.009098 57.404) (end 106.426 57.404) (width 0.25) (layer F.Cu) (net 15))
 (segment (start 103.273956 70.472143) (end 102.976899 70.175086) (width 0.25) (layer F.Cu) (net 15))
 (segment (start 103.69822 70.472143) (end 103.273956 70.472143) (width 0.25) (layer F.Cu) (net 15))
 (segment (start 102.976899 70.175086) (end 102.976899 64.897) (width 0.25) (layer F.Cu) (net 15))
 (segment (start 102.976899 64.897) (end 102.963699 64.8838) (width 0.25) (layer F.Cu) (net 15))
 (segment (start 102.963699 64.8838) (end 102.963699 58.449399) (width 0.25) (layer F.Cu) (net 15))
 (segment (start 102.963699 58.449399) (end 104.009098 57.404) (width 0.25) (layer F.Cu) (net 15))
 (segment (start 115.1255 80.9879) (end 115.1255 82.2379) (width 0.25) (layer F.Cu) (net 4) (status 10))
 (segment (start 115.1255 82.2379) (end 115.050499 82.312901) (width 0.25) (layer F.Cu) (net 4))
 (segment (start 115.050499 82.312901) (end 104.469499 82.312901) (width 0.25) (layer F.Cu) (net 4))
 (segment (start 104.469499 82.312901) (end 103.780499 81.623901) (width 0.25) (layer F.Cu) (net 4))
 (segment (start 103.780499 81.623901) (end 103.780499 78.907101) (width 0.25) (layer F.Cu) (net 4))
 (segment (start 103.780499 78.907101) (end 108.1218 74.5658) (width 0.25) (layer F.Cu) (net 4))
 (segment (start 108.1218 74.5658) (end 108.1218 73.5158) (width 0.25) (layer F.Cu) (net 4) (status 20))
 (segment (start 109.7218 72.4658) (end 110.29018 71.89742) (width 0.25) (layer F.Cu) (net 5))
 (segment (start 109.7218 73.5158) (end 109.7218 72.4658) (width 0.25) (layer F.Cu) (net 5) (status 10))
 (segment (start 112.6055 74.16532) (end 110.3376 71.89742) (width 0.25) (layer B.Cu) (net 5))
 (segment (start 112.6055 80.9879) (end 112.6055 74.16532) (width 0.25) (layer B.Cu) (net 5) (status 10))
 (segment (start 110.29018 71.89742) (end 110.3376 71.89742) (width 0.25) (layer F.Cu) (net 5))
 (via (at 110.3376 71.89742) (size 0.6) (drill 0.4) (layers F.Cu B.Cu) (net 5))
 (segment (start 110.5218 73.5158) (end 110.5218 74.5658) (width 0.25) (layer F.Cu) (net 6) (status 10))
 (segment (start 110.5218 74.5658) (end 110.291201 74.796399) (width 0.25) (layer F.Cu) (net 6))
 (segment (start 110.291201 74.796399) (end 109.515999 74.796399) (width 0.25) (layer F.Cu) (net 6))
 (segment (start 109.515999 74.796399) (end 109.450999 74.861399) (width 0.25) (layer F.Cu) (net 6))
 (segment (start 109.450999 74.861399) (end 109.450999 78.919186) (width 0.25) (layer F.Cu) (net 6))
 (segment (start 109.450999 78.919186) (end 110.1055 79.573687) (width 0.25) (layer F.Cu) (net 6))
 (segment (start 110.1055 79.573687) (end 110.1055 80.9879) (width 0.25) (layer F.Cu) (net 6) (status 20))
 (segment (start 108.9218 73.5158) (end 108.9218 77.1716) (width 0.25) (layer F.Cu) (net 7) (status 10))
 (segment (start 108.9218 77.1716) (end 105.1055 80.9879) (width 0.25) (layer F.Cu) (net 7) (status 20))
 (segment (start 120.523328 75.941816) (end 120.823327 75.641817) (width 0.25) (layer B.Cu) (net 13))
 (segment (start 120.351343 76.113801) (end 120.523328 75.941816) (width 0.25) (layer B.Cu) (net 13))
 (segment (start 118.227001 76.113801) (end 120.351343 76.113801) (width 0.25) (layer B.Cu) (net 13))
 (segment (start 109.519999 67.305199) (end 109.519999 67.406799) (width 0.25) (layer B.Cu) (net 13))
 (segment (start 109.519999 67.406799) (end 118.227001 76.113801) (width 0.25) (layer B.Cu) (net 13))
 (segment (start 109.22 67.0052) (end 109.519999 67.305199) (width 0.25) (layer B.Cu) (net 13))
 (segment (start 121.123326 75.341818) (end 120.823327 75.641817) (width 0.25) (layer F.Cu) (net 13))
 (via (at 120.823327 75.641817) (size 0.6) (drill 0.4) (layers F.Cu B.Cu) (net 13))
 (segment (start 125.3236 78.5368) (end 122.128618 75.341818) (width 0.25) (layer F.Cu) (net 13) (status 10))
 (segment (start 122.128618 75.341818) (end 121.123326 75.341818) (width 0.25) (layer F.Cu) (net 13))
 (segment (start 108.1218 65.0158) (end 108.1218 66.0658) (width 0.25) (layer F.Cu) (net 13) (status 10))
 (segment (start 108.1218 66.0658) (end 109.0612 67.0052) (width 0.25) (layer F.Cu) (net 13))
 (segment (start 109.0612 67.0052) (end 109.22 67.0052) (width 0.25) (layer F.Cu) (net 13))
 (via (at 109.22 67.0052) (size 0.6) (drill 0.4) (layers F.Cu B.Cu) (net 13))
 (segment (start 121.03272 76.563812) (end 121.089022 76.50751) (width 0.25) (layer B.Cu) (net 14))
 (segment (start 121.089022 76.50751) (end 121.389021 76.207511) (width 0.25) (layer B.Cu) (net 14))
 (segment (start 122.7836 78.5368) (end 122.7836 77.334719) (width 0.25) (layer F.Cu) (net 14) (status 10))
 (segment (start 108.580732 67.751357) (end 109.228146 67.751357) (width 0.25) (layer B.Cu) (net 14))
 (segment (start 109.228146 67.751357) (end 118.040601 76.563812) (width 0.25) (layer B.Cu) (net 14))
 (segment (start 122.7836 77.334719) (end 121.656392 76.207511) (width 0.25) (layer F.Cu) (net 14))
 (via (at 121.389021 76.207511) (size 0.6) (drill 0.4) (layers F.Cu B.Cu) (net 14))
 (segment (start 118.040601 76.563812) (end 121.03272 76.563812) (width 0.25) (layer B.Cu) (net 14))
 (segment (start 121.656392 76.207511) (end 121.389021 76.207511) (width 0.25) (layer F.Cu) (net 14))
 (via (at 108.580732 67.751357) (size 0.6) (drill 0.4) (layers F.Cu B.Cu) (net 14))
 (segment (start 106.6718 66.4658) (end 107.7218 66.4658) (width 0.25) (layer F.Cu) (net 14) (status 10))
 (segment (start 107.7218 66.4658) (end 108.580732 67.324732) (width 0.25) (layer F.Cu) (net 14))
 (segment (start 108.580732 67.324732) (end 108.580732 67.327093) (width 0.25) (layer F.Cu) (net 14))
 (segment (start 108.580732 67.327093) (end 108.580732 67.751357) (width 0.25) (layer F.Cu) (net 14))
 (segment (start 106.6718 66.4658) (end 107.440162 66.4658) (width 0.25) (layer F.Cu) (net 14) (status 30))
 (segment (start 110.7948 67.4116) (end 109.524001 66.140801) (width 0.25) (layer F.Cu) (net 12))
 (segment (start 109.524001 66.140801) (end 108.996801 66.140801) (width 0.25) (layer F.Cu) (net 12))
 (segment (start 108.996801 66.140801) (end 108.9218 66.0658) (width 0.25) (layer F.Cu) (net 12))
 (segment (start 108.9218 66.0658) (end 108.9218 65.0158) (width 0.25) (layer F.Cu) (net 12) (status 20))
 (segment (start 111.3028 67.4116) (end 110.7948 67.4116) (width 0.25) (layer F.Cu) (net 12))
 (segment (start 119.6848 75.4888) (end 111.6076 67.4116) (width 0.25) (layer B.Cu) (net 12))
 (segment (start 111.6076 67.4116) (end 111.3028 67.4116) (width 0.25) (layer B.Cu) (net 12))
 (via (at 111.3028 67.4116) (size 0.6) (drill 0.4) (layers F.Cu B.Cu) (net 12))
 (segment (start 121.608599 79.901799) (end 121.608599 77.412599) (width 0.25) (layer F.Cu) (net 12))
 (segment (start 122.7836 81.0768) (end 121.608599 79.901799) (width 0.25) (layer F.Cu) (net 12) (status 10))
 (segment (start 121.608599 77.412599) (end 119.6848 75.4888) (width 0.25) (layer F.Cu) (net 12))
 (via (at 119.6848 75.4888) (size 0.6) (drill 0.4) (layers F.Cu B.Cu) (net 12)))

